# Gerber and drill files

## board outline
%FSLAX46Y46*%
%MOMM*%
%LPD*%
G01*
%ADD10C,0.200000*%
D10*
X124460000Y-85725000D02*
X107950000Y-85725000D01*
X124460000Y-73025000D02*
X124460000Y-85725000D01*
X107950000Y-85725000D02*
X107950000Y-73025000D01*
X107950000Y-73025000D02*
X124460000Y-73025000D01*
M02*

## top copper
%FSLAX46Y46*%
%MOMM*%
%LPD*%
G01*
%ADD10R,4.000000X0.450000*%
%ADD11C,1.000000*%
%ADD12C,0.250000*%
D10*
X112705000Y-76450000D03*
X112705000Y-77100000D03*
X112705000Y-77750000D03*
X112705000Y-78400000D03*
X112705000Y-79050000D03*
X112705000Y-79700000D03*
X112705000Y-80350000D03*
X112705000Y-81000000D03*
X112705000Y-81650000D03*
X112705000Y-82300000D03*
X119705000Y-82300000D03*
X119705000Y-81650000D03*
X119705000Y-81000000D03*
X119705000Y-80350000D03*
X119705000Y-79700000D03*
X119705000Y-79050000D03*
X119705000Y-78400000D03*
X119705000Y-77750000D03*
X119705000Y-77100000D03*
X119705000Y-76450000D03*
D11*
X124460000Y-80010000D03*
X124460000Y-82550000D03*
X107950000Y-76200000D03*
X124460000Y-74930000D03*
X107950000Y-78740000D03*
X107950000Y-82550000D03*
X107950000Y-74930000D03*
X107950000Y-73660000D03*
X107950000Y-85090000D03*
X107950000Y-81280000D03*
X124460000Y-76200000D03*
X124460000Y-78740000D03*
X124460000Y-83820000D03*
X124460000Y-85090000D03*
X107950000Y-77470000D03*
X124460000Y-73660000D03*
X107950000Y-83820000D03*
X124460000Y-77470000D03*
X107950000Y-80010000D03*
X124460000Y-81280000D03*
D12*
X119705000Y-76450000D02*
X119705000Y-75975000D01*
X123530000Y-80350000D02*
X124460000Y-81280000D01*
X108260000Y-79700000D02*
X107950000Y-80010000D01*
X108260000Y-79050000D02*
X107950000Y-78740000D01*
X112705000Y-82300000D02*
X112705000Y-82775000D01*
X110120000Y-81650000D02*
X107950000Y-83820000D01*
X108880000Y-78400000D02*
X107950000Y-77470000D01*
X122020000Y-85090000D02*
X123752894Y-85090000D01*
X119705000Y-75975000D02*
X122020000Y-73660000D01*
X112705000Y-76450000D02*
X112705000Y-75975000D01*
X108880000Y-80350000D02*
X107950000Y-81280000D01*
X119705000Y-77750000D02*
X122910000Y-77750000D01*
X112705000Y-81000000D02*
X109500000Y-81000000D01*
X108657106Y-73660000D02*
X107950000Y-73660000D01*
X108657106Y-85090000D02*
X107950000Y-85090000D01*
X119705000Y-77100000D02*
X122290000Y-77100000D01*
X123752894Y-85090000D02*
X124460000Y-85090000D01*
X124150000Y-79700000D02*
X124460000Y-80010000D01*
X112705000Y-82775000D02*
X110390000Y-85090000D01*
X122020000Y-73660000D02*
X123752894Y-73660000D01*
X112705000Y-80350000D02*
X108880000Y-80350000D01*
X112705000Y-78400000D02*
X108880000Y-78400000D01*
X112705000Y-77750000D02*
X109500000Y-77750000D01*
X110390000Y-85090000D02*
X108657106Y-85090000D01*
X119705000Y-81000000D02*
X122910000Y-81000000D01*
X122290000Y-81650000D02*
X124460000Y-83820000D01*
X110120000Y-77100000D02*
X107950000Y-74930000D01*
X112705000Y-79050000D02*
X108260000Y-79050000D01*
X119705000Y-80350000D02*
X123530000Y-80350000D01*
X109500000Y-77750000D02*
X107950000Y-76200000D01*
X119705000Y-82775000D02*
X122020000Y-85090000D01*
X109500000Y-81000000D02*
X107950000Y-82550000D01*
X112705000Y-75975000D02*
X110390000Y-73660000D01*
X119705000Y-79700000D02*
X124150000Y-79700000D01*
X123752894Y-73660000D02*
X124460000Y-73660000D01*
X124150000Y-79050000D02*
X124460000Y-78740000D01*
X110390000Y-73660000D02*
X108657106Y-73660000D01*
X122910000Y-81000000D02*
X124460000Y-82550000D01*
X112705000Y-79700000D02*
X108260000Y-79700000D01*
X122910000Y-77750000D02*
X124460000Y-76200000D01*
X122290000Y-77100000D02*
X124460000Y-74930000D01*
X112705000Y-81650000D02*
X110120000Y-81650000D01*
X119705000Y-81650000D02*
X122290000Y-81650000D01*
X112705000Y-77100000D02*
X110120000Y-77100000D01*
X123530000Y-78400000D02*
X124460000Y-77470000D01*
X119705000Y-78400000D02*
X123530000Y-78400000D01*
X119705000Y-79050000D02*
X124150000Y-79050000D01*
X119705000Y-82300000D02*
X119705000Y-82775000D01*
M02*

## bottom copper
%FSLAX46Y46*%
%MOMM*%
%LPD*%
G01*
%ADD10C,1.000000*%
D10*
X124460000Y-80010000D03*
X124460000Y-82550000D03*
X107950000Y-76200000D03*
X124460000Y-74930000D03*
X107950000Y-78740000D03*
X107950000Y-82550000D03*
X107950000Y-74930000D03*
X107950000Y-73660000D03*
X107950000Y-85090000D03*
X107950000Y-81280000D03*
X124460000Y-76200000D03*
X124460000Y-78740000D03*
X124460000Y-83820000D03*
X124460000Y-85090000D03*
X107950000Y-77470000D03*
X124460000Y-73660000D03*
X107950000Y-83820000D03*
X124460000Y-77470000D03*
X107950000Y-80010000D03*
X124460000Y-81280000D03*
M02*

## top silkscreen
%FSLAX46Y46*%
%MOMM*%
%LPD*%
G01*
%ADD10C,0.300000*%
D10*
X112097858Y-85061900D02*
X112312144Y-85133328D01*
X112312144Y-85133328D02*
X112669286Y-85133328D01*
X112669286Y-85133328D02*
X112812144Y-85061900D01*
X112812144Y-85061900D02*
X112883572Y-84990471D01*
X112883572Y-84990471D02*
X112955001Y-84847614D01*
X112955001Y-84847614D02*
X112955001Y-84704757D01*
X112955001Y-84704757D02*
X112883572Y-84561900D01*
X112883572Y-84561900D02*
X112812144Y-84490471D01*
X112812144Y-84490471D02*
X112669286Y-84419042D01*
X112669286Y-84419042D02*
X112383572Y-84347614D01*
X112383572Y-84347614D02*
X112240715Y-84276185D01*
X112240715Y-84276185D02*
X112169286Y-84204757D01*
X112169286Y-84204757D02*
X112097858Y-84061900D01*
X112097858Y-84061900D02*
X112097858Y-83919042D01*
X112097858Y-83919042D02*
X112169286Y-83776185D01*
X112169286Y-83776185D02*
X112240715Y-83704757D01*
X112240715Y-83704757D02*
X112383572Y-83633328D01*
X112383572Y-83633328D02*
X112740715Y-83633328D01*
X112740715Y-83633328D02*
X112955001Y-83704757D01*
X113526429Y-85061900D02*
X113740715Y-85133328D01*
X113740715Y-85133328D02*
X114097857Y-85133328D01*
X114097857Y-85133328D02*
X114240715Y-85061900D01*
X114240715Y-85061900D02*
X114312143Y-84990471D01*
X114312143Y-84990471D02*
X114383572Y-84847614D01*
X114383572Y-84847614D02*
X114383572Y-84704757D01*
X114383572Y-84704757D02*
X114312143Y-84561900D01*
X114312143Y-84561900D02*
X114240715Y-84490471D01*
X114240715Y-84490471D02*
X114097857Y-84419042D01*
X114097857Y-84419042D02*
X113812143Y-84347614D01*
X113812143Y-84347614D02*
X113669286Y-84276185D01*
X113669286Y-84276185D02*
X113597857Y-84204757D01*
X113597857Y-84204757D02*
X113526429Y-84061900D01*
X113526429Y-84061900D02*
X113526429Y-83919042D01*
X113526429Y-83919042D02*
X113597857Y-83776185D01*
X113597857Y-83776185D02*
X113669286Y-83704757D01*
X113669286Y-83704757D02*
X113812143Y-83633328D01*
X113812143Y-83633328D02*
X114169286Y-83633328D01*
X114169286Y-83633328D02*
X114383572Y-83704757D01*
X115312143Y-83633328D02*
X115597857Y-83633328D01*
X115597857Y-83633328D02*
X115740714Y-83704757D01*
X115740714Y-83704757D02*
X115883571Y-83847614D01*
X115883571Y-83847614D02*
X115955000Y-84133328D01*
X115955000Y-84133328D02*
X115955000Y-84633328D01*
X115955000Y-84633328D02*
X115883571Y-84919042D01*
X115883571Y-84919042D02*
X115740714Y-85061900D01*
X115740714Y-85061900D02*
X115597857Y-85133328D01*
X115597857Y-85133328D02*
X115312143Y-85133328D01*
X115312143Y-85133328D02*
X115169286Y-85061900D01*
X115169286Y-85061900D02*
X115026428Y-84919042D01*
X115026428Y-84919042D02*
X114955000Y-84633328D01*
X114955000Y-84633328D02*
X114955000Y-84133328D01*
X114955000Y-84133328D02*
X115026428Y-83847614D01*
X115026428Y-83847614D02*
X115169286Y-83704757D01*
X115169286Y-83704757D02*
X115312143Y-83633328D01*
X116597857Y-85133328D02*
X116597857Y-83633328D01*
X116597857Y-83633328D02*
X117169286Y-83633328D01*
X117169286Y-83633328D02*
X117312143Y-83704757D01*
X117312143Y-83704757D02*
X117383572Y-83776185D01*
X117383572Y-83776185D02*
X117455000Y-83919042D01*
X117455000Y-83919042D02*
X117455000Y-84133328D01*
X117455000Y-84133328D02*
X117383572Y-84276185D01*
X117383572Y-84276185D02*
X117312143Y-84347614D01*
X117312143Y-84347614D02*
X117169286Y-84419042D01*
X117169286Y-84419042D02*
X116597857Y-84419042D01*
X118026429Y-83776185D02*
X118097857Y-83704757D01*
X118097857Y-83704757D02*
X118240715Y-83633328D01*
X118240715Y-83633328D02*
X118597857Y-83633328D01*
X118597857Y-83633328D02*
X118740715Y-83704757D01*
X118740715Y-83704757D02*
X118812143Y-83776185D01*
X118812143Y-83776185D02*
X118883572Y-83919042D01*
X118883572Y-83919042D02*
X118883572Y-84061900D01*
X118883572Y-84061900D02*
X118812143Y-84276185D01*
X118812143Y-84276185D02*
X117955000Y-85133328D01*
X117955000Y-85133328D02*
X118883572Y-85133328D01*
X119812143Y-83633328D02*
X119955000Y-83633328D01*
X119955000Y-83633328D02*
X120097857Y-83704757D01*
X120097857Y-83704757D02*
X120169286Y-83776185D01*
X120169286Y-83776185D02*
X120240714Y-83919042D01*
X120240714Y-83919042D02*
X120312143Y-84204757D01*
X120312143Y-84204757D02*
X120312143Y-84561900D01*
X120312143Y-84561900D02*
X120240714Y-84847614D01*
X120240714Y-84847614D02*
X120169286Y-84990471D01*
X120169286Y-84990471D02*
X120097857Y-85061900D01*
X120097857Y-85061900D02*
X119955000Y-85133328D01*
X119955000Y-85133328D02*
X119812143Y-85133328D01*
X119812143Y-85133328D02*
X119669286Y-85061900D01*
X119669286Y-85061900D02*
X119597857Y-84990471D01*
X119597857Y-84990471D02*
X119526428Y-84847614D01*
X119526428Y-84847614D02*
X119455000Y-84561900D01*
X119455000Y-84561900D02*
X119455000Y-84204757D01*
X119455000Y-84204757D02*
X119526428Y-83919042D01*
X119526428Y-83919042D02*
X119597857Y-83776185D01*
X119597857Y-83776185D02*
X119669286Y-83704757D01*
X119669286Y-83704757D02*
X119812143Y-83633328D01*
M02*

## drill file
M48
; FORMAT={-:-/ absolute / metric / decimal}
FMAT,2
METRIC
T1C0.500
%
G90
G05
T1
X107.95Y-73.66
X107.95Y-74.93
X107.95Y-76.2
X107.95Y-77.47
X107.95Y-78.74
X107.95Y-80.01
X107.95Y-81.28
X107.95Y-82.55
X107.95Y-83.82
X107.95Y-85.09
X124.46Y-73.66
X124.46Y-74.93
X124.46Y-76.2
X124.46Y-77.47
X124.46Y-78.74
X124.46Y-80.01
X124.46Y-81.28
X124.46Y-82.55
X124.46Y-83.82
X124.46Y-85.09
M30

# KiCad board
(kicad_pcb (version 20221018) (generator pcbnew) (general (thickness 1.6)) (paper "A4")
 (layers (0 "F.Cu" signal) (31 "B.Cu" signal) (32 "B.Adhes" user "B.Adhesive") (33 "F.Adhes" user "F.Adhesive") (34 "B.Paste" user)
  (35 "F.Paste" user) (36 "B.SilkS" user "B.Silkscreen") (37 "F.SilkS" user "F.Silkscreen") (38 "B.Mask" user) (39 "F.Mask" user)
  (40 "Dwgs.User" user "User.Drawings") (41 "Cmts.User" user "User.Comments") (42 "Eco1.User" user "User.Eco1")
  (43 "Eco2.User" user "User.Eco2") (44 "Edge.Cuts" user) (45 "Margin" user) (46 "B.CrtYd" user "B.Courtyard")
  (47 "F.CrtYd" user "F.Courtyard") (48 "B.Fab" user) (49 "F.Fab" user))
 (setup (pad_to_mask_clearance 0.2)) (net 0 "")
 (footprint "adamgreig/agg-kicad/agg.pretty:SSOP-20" (layer "F.Cu") (at 116.205 79.375)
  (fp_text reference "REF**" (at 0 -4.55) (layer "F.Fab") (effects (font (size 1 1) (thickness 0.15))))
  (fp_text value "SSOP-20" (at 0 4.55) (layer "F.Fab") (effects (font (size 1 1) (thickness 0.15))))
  (pad "1" smd rect (at -3.5 -2.925) (size 4 0.45) (layers "F.Cu" "F.Paste" "F.Mask"))
  (pad "2" smd rect (at -3.5 -2.275) (size 4 0.45) (layers "F.Cu" "F.Paste" "F.Mask"))
  (pad "3" smd rect (at -3.5 -1.625) (size 4 0.45) (layers "F.Cu" "F.Paste" "F.Mask"))
  (pad "4" smd rect (at -3.5 -0.975) (size 4 0.45) (layers "F.Cu" "F.Paste" "F.Mask"))
  (pad "5" smd rect (at -3.5 -0.325) (size 4 0.45) (layers "F.Cu" "F.Paste" "F.Mask"))
  (pad "6" smd rect (at -3.5 0.325) (size 4 0.45) (layers "F.Cu" "F.Paste" "F.Mask"))
  (pad "7" smd rect (at -3.5 0.975) (size 4 0.45) (layers "F.Cu" "F.Paste" "F.Mask"))
  (pad "8" smd rect (at -3.5 1.625) (size 4 0.45) (layers "F.Cu" "F.Paste" "F.Mask"))
  (pad "9" smd rect (at -3.5 2.275) (size 4 0.45) (layers "F.Cu" "F.Paste" "F.Mask"))
  (pad "10" smd rect (at -3.5 2.925) (size 4 0.45) (layers "F.Cu" "F.Paste" "F.Mask"))
  (pad "11" smd rect (at 3.5 2.925) (size 4 0.45) (layers "F.Cu" "F.Paste" "F.Mask"))
  (pad "12" smd rect (at 3.5 2.275) (size 4 0.45) (layers "F.Cu" "F.Paste" "F.Mask"))
  (pad "13" smd rect (at 3.5 1.625) (size 4 0.45) (layers "F.Cu" "F.Paste" "F.Mask"))
  (pad "14" smd rect (at 3.5 0.975) (size 4 0.45) (layers "F.Cu" "F.Paste" "F.Mask"))
  (pad "15" smd rect (at 3.5 0.325) (size 4 0.45) (layers "F.Cu" "F.Paste" "F.Mask"))
  (pad "16" smd rect (at 3.5 -0.325) (size 4 0.45) (layers "F.Cu" "F.Paste" "F.Mask"))
  (pad "17" smd rect (at 3.5 -0.975) (size 4 0.45) (layers "F.Cu" "F.Paste" "F.Mask"))
  (pad "18" smd rect (at 3.5 -1.625) (size 4 0.45) (layers "F.Cu" "F.Paste" "F.Mask"))
  (pad "19" smd rect (at 3.5 -2.275) (size 4 0.45) (layers "F.Cu" "F.Paste" "F.Mask"))
  (pad "20" smd rect (at 3.5 -2.925) (size 4 0.45) (layers "F.Cu" "F.Paste" "F.Mask")))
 (gr_line (start 124.46 85.725) (end 107.95 85.725) (stroke (width 0.2) (type solid)) (layer "Edge.Cuts"))
 (gr_line (start 124.46 73.025) (end 124.46 85.725) (stroke (width 0.2) (type solid)) (layer "Edge.Cuts"))
 (gr_line (start 107.95 85.725) (end 107.95 73.025) (stroke (width 0.2) (type solid)) (layer "Edge.Cuts"))
 (gr_line (start 107.95 73.025) (end 124.46 73.025) (stroke (width 0.2) (type solid)) (layer "Edge.Cuts"))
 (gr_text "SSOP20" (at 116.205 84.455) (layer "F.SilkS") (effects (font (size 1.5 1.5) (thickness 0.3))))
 (segment (start 119.705 76.45) (end 119.705 75.975) (width 0.25) (layer "F.Cu") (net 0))
 (segment (start 123.53 80.35) (end 124.46 81.28) (width 0.25) (layer "F.Cu") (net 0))
 (segment (start 108.26 79.7) (end 107.95 80.01) (width 0.25) (layer "F.Cu") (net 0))
 (segment (start 108.26 79.05) (end 107.95 78.74) (width 0.25) (layer "F.Cu") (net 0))
 (segment (start 112.705 82.3) (end 112.705 82.775) (width 0.25) (layer "F.Cu") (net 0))
 (segment (start 110.12 81.65) (end 107.95 83.82) (width 0.25) (layer "F.Cu") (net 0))
 (segment (start 108.88 78.4) (end 107.95 77.47) (width 0.25) (layer "F.Cu") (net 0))
 (segment (start 122.02 85.09) (end 123.752894 85.09) (width 0.25) (layer "F.Cu") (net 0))
 (segment (start 119.705 75.975) (end 122.02 73.66) (width 0.25) (layer "F.Cu") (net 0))
 (segment (start 112.705 76.45) (end 112.705 75.975) (width 0.25) (layer "F.Cu") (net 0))
 (segment (start 108.88 80.35) (end 107.95 81.28) (width 0.25) (layer "F.Cu") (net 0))
 (segment (start 119.705 77.75) (end 122.91 77.75) (width 0.25) (layer "F.Cu") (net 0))
 (segment (start 112.705 81) (end 109.5 81) (width 0.25) (layer "F.Cu") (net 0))
 (segment (start 108.657106 73.66) (end 107.95 73.66) (width 0.25) (layer "F.Cu") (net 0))
 (segment (start 108.657106 85.09) (end 107.95 85.09) (width 0.25) (layer "F.Cu") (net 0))
 (segment (start 119.705 77.1) (end 122.29 77.1) (width 0.25) (layer "F.Cu") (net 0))
 (segment (start 123.752894 85.09) (end 124.46 85.09) (width 0.25) (layer "F.Cu") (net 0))
 (segment (start 124.15 79.7) (end 124.46 80.01) (width 0.25) (layer "F.Cu") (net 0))
 (segment (start 112.705 82.775) (end 110.39 85.09) (width 0.25) (layer "F.Cu") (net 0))
 (segment (start 122.02 73.66) (end 123.752894 73.66) (width 0.25) (layer "F.Cu") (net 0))
 (segment (start 112.705 80.35) (end 108.88 80.35) (width 0.25) (layer "F.Cu") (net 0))
 (segment (start 112.705 78.4) (end 108.88 78.4) (width 0.25) (layer "F.Cu") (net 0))
 (segment (start 112.705 77.75) (end 109.5 77.75) (width 0.25) (layer "F.Cu") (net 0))
 (segment (start 110.39 85.09) (end 108.657106 85.09) (width 0.25) (layer "F.Cu") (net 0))
 (segment (start 119.705 81) (end 122.91 81) (width 0.25) (layer "F.Cu") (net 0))
 (segment (start 122.29 81.65) (end 124.46 83.82) (width 0.25) (layer "F.Cu") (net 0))
 (segment (start 110.12 77.1) (end 107.95 74.93) (width 0.25) (layer "F.Cu") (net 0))
 (segment (start 112.705 79.05) (end 108.26 79.05) (width 0.25) (layer "F.Cu") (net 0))
 (segment (start 119.705 80.35) (end 123.53 80.35) (width 0.25) (layer "F.Cu") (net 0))
 (segment (start 109.5 77.75) (end 107.95 76.2) (width 0.25) (layer "F.Cu") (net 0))
 (segment (start 119.705 82.775) (end 122.02 85.09) (width 0.25) (layer "F.Cu") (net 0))
 (segment (start 109.5 81) (end 107.95 82.55) (width 0.25) (layer "F.Cu") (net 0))
 (segment (start 112.705 75.975) (end 110.39 73.66) (width 0.25) (layer "F.Cu") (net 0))
 (segment (start 119.705 79.7) (end 124.15 79.7) (width 0.25) (layer "F.Cu") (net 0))
 (segment (start 123.752894 73.66) (end 124.46 73.66) (width 0.25) (layer "F.Cu") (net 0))
 (segment (start 124.15 79.05) (end 124.46 78.74) (width 0.25) (layer "F.Cu") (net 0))
 (segment (start 110.39 73.66) (end 108.657106 73.66) (width 0.25) (layer "F.Cu") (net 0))
 (segment (start 122.91 81) (end 124.46 82.55) (width 0.25) (layer "F.Cu") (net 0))
 (segment (start 112.705 79.7) (end 108.26 79.7) (width 0.25) (layer "F.Cu") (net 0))
 (segment (start 122.91 77.75) (end 124.46 76.2) (width 0.25) (layer "F.Cu") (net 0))
 (segment (start 122.29 77.1) (end 124.46 74.93) (width 0.25) (layer "F.Cu") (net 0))
 (segment (start 112.705 81.65) (end 110.12 81.65) (width 0.25) (layer "F.Cu") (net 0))
 (segment (start 119.705 81.65) (end 122.29 81.65) (width 0.25) (layer "F.Cu") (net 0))
 (segment (start 112.705 77.1) (end 110.12 77.1) (width 0.25) (layer "F.Cu") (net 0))
 (segment (start 123.53 78.4) (end 124.46 77.47) (width 0.25) (layer "F.Cu") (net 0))
 (segment (start 119.705 78.4) (end 123.53 78.4) (width 0.25) (layer "F.Cu") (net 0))
 (segment (start 119.705 79.05) (end 124.15 79.05) (width 0.25) (layer "F.Cu") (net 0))
 (segment (start 119.705 82.3) (end 119.705 82.775) (width 0.25) (layer "F.Cu") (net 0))
 (via (at 124.46 80.01) (size 1) (drill 0.5) (layers "F.Cu" "B.Cu") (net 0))
 (via (at 124.46 82.55) (size 1) (drill 0.5) (layers "F.Cu" "B.Cu") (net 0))
 (via (at 107.95 76.2) (size 1) (drill 0.5) (layers "F.Cu" "B.Cu") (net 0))
 (via (at 124.46 74.93) (size 1) (drill 0.5) (layers "F.Cu" "B.Cu") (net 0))
 (via (at 107.95 78.74) (size 1) (drill 0.5) (layers "F.Cu" "B.Cu") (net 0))
 (via (at 107.95 82.55) (size 1) (drill 0.5) (layers "F.Cu" "B.Cu") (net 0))
 (via (at 107.95 74.93) (size 1) (drill 0.5) (layers "F.Cu" "B.Cu") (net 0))
 (via (at 107.95 73.66) (size 1) (drill 0.5) (layers "F.Cu" "B.Cu") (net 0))
 (via (at 107.95 85.09) (size 1) (drill 0.5) (layers "F.Cu" "B.Cu") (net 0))
 (via (at 107.95 81.28) (size 1) (drill 0.5) (layers "F.Cu" "B.Cu") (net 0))
 (via (at 124.46 76.2) (size 1) (drill 0.5) (layers "F.Cu" "B.Cu") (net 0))
 (via (at 124.46 78.74) (size 1) (drill 0.5) (layers "F.Cu" "B.Cu") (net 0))
 (via (at 124.46 83.82) (size 1) (drill 0.5) (layers "F.Cu" "B.Cu") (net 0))
 (via (at 124.46 85.09) (size 1) (drill 0.5) (layers "F.Cu" "B.Cu") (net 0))
 (via (at 107.95 77.47) (size 1) (drill 0.5) (layers "F.Cu" "B.Cu") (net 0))
 (via (at 124.46 73.66) (size 1) (drill 0.5) (layers "F.Cu" "B.Cu") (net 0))
 (via (at 107.95 83.82) (size 1) (drill 0.5) (layers "F.Cu" "B.Cu") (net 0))
 (via (at 124.46 77.47) (size 1) (drill 0.5) (layers "F.Cu" "B.Cu") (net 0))
 (via (at 107.95 80.01) (size 1) (drill 0.5) (layers "F.Cu" "B.Cu") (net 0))
 (via (at 124.46 81.28) (size 1) (drill 0.5) (layers "F.Cu" "B.Cu") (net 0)))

